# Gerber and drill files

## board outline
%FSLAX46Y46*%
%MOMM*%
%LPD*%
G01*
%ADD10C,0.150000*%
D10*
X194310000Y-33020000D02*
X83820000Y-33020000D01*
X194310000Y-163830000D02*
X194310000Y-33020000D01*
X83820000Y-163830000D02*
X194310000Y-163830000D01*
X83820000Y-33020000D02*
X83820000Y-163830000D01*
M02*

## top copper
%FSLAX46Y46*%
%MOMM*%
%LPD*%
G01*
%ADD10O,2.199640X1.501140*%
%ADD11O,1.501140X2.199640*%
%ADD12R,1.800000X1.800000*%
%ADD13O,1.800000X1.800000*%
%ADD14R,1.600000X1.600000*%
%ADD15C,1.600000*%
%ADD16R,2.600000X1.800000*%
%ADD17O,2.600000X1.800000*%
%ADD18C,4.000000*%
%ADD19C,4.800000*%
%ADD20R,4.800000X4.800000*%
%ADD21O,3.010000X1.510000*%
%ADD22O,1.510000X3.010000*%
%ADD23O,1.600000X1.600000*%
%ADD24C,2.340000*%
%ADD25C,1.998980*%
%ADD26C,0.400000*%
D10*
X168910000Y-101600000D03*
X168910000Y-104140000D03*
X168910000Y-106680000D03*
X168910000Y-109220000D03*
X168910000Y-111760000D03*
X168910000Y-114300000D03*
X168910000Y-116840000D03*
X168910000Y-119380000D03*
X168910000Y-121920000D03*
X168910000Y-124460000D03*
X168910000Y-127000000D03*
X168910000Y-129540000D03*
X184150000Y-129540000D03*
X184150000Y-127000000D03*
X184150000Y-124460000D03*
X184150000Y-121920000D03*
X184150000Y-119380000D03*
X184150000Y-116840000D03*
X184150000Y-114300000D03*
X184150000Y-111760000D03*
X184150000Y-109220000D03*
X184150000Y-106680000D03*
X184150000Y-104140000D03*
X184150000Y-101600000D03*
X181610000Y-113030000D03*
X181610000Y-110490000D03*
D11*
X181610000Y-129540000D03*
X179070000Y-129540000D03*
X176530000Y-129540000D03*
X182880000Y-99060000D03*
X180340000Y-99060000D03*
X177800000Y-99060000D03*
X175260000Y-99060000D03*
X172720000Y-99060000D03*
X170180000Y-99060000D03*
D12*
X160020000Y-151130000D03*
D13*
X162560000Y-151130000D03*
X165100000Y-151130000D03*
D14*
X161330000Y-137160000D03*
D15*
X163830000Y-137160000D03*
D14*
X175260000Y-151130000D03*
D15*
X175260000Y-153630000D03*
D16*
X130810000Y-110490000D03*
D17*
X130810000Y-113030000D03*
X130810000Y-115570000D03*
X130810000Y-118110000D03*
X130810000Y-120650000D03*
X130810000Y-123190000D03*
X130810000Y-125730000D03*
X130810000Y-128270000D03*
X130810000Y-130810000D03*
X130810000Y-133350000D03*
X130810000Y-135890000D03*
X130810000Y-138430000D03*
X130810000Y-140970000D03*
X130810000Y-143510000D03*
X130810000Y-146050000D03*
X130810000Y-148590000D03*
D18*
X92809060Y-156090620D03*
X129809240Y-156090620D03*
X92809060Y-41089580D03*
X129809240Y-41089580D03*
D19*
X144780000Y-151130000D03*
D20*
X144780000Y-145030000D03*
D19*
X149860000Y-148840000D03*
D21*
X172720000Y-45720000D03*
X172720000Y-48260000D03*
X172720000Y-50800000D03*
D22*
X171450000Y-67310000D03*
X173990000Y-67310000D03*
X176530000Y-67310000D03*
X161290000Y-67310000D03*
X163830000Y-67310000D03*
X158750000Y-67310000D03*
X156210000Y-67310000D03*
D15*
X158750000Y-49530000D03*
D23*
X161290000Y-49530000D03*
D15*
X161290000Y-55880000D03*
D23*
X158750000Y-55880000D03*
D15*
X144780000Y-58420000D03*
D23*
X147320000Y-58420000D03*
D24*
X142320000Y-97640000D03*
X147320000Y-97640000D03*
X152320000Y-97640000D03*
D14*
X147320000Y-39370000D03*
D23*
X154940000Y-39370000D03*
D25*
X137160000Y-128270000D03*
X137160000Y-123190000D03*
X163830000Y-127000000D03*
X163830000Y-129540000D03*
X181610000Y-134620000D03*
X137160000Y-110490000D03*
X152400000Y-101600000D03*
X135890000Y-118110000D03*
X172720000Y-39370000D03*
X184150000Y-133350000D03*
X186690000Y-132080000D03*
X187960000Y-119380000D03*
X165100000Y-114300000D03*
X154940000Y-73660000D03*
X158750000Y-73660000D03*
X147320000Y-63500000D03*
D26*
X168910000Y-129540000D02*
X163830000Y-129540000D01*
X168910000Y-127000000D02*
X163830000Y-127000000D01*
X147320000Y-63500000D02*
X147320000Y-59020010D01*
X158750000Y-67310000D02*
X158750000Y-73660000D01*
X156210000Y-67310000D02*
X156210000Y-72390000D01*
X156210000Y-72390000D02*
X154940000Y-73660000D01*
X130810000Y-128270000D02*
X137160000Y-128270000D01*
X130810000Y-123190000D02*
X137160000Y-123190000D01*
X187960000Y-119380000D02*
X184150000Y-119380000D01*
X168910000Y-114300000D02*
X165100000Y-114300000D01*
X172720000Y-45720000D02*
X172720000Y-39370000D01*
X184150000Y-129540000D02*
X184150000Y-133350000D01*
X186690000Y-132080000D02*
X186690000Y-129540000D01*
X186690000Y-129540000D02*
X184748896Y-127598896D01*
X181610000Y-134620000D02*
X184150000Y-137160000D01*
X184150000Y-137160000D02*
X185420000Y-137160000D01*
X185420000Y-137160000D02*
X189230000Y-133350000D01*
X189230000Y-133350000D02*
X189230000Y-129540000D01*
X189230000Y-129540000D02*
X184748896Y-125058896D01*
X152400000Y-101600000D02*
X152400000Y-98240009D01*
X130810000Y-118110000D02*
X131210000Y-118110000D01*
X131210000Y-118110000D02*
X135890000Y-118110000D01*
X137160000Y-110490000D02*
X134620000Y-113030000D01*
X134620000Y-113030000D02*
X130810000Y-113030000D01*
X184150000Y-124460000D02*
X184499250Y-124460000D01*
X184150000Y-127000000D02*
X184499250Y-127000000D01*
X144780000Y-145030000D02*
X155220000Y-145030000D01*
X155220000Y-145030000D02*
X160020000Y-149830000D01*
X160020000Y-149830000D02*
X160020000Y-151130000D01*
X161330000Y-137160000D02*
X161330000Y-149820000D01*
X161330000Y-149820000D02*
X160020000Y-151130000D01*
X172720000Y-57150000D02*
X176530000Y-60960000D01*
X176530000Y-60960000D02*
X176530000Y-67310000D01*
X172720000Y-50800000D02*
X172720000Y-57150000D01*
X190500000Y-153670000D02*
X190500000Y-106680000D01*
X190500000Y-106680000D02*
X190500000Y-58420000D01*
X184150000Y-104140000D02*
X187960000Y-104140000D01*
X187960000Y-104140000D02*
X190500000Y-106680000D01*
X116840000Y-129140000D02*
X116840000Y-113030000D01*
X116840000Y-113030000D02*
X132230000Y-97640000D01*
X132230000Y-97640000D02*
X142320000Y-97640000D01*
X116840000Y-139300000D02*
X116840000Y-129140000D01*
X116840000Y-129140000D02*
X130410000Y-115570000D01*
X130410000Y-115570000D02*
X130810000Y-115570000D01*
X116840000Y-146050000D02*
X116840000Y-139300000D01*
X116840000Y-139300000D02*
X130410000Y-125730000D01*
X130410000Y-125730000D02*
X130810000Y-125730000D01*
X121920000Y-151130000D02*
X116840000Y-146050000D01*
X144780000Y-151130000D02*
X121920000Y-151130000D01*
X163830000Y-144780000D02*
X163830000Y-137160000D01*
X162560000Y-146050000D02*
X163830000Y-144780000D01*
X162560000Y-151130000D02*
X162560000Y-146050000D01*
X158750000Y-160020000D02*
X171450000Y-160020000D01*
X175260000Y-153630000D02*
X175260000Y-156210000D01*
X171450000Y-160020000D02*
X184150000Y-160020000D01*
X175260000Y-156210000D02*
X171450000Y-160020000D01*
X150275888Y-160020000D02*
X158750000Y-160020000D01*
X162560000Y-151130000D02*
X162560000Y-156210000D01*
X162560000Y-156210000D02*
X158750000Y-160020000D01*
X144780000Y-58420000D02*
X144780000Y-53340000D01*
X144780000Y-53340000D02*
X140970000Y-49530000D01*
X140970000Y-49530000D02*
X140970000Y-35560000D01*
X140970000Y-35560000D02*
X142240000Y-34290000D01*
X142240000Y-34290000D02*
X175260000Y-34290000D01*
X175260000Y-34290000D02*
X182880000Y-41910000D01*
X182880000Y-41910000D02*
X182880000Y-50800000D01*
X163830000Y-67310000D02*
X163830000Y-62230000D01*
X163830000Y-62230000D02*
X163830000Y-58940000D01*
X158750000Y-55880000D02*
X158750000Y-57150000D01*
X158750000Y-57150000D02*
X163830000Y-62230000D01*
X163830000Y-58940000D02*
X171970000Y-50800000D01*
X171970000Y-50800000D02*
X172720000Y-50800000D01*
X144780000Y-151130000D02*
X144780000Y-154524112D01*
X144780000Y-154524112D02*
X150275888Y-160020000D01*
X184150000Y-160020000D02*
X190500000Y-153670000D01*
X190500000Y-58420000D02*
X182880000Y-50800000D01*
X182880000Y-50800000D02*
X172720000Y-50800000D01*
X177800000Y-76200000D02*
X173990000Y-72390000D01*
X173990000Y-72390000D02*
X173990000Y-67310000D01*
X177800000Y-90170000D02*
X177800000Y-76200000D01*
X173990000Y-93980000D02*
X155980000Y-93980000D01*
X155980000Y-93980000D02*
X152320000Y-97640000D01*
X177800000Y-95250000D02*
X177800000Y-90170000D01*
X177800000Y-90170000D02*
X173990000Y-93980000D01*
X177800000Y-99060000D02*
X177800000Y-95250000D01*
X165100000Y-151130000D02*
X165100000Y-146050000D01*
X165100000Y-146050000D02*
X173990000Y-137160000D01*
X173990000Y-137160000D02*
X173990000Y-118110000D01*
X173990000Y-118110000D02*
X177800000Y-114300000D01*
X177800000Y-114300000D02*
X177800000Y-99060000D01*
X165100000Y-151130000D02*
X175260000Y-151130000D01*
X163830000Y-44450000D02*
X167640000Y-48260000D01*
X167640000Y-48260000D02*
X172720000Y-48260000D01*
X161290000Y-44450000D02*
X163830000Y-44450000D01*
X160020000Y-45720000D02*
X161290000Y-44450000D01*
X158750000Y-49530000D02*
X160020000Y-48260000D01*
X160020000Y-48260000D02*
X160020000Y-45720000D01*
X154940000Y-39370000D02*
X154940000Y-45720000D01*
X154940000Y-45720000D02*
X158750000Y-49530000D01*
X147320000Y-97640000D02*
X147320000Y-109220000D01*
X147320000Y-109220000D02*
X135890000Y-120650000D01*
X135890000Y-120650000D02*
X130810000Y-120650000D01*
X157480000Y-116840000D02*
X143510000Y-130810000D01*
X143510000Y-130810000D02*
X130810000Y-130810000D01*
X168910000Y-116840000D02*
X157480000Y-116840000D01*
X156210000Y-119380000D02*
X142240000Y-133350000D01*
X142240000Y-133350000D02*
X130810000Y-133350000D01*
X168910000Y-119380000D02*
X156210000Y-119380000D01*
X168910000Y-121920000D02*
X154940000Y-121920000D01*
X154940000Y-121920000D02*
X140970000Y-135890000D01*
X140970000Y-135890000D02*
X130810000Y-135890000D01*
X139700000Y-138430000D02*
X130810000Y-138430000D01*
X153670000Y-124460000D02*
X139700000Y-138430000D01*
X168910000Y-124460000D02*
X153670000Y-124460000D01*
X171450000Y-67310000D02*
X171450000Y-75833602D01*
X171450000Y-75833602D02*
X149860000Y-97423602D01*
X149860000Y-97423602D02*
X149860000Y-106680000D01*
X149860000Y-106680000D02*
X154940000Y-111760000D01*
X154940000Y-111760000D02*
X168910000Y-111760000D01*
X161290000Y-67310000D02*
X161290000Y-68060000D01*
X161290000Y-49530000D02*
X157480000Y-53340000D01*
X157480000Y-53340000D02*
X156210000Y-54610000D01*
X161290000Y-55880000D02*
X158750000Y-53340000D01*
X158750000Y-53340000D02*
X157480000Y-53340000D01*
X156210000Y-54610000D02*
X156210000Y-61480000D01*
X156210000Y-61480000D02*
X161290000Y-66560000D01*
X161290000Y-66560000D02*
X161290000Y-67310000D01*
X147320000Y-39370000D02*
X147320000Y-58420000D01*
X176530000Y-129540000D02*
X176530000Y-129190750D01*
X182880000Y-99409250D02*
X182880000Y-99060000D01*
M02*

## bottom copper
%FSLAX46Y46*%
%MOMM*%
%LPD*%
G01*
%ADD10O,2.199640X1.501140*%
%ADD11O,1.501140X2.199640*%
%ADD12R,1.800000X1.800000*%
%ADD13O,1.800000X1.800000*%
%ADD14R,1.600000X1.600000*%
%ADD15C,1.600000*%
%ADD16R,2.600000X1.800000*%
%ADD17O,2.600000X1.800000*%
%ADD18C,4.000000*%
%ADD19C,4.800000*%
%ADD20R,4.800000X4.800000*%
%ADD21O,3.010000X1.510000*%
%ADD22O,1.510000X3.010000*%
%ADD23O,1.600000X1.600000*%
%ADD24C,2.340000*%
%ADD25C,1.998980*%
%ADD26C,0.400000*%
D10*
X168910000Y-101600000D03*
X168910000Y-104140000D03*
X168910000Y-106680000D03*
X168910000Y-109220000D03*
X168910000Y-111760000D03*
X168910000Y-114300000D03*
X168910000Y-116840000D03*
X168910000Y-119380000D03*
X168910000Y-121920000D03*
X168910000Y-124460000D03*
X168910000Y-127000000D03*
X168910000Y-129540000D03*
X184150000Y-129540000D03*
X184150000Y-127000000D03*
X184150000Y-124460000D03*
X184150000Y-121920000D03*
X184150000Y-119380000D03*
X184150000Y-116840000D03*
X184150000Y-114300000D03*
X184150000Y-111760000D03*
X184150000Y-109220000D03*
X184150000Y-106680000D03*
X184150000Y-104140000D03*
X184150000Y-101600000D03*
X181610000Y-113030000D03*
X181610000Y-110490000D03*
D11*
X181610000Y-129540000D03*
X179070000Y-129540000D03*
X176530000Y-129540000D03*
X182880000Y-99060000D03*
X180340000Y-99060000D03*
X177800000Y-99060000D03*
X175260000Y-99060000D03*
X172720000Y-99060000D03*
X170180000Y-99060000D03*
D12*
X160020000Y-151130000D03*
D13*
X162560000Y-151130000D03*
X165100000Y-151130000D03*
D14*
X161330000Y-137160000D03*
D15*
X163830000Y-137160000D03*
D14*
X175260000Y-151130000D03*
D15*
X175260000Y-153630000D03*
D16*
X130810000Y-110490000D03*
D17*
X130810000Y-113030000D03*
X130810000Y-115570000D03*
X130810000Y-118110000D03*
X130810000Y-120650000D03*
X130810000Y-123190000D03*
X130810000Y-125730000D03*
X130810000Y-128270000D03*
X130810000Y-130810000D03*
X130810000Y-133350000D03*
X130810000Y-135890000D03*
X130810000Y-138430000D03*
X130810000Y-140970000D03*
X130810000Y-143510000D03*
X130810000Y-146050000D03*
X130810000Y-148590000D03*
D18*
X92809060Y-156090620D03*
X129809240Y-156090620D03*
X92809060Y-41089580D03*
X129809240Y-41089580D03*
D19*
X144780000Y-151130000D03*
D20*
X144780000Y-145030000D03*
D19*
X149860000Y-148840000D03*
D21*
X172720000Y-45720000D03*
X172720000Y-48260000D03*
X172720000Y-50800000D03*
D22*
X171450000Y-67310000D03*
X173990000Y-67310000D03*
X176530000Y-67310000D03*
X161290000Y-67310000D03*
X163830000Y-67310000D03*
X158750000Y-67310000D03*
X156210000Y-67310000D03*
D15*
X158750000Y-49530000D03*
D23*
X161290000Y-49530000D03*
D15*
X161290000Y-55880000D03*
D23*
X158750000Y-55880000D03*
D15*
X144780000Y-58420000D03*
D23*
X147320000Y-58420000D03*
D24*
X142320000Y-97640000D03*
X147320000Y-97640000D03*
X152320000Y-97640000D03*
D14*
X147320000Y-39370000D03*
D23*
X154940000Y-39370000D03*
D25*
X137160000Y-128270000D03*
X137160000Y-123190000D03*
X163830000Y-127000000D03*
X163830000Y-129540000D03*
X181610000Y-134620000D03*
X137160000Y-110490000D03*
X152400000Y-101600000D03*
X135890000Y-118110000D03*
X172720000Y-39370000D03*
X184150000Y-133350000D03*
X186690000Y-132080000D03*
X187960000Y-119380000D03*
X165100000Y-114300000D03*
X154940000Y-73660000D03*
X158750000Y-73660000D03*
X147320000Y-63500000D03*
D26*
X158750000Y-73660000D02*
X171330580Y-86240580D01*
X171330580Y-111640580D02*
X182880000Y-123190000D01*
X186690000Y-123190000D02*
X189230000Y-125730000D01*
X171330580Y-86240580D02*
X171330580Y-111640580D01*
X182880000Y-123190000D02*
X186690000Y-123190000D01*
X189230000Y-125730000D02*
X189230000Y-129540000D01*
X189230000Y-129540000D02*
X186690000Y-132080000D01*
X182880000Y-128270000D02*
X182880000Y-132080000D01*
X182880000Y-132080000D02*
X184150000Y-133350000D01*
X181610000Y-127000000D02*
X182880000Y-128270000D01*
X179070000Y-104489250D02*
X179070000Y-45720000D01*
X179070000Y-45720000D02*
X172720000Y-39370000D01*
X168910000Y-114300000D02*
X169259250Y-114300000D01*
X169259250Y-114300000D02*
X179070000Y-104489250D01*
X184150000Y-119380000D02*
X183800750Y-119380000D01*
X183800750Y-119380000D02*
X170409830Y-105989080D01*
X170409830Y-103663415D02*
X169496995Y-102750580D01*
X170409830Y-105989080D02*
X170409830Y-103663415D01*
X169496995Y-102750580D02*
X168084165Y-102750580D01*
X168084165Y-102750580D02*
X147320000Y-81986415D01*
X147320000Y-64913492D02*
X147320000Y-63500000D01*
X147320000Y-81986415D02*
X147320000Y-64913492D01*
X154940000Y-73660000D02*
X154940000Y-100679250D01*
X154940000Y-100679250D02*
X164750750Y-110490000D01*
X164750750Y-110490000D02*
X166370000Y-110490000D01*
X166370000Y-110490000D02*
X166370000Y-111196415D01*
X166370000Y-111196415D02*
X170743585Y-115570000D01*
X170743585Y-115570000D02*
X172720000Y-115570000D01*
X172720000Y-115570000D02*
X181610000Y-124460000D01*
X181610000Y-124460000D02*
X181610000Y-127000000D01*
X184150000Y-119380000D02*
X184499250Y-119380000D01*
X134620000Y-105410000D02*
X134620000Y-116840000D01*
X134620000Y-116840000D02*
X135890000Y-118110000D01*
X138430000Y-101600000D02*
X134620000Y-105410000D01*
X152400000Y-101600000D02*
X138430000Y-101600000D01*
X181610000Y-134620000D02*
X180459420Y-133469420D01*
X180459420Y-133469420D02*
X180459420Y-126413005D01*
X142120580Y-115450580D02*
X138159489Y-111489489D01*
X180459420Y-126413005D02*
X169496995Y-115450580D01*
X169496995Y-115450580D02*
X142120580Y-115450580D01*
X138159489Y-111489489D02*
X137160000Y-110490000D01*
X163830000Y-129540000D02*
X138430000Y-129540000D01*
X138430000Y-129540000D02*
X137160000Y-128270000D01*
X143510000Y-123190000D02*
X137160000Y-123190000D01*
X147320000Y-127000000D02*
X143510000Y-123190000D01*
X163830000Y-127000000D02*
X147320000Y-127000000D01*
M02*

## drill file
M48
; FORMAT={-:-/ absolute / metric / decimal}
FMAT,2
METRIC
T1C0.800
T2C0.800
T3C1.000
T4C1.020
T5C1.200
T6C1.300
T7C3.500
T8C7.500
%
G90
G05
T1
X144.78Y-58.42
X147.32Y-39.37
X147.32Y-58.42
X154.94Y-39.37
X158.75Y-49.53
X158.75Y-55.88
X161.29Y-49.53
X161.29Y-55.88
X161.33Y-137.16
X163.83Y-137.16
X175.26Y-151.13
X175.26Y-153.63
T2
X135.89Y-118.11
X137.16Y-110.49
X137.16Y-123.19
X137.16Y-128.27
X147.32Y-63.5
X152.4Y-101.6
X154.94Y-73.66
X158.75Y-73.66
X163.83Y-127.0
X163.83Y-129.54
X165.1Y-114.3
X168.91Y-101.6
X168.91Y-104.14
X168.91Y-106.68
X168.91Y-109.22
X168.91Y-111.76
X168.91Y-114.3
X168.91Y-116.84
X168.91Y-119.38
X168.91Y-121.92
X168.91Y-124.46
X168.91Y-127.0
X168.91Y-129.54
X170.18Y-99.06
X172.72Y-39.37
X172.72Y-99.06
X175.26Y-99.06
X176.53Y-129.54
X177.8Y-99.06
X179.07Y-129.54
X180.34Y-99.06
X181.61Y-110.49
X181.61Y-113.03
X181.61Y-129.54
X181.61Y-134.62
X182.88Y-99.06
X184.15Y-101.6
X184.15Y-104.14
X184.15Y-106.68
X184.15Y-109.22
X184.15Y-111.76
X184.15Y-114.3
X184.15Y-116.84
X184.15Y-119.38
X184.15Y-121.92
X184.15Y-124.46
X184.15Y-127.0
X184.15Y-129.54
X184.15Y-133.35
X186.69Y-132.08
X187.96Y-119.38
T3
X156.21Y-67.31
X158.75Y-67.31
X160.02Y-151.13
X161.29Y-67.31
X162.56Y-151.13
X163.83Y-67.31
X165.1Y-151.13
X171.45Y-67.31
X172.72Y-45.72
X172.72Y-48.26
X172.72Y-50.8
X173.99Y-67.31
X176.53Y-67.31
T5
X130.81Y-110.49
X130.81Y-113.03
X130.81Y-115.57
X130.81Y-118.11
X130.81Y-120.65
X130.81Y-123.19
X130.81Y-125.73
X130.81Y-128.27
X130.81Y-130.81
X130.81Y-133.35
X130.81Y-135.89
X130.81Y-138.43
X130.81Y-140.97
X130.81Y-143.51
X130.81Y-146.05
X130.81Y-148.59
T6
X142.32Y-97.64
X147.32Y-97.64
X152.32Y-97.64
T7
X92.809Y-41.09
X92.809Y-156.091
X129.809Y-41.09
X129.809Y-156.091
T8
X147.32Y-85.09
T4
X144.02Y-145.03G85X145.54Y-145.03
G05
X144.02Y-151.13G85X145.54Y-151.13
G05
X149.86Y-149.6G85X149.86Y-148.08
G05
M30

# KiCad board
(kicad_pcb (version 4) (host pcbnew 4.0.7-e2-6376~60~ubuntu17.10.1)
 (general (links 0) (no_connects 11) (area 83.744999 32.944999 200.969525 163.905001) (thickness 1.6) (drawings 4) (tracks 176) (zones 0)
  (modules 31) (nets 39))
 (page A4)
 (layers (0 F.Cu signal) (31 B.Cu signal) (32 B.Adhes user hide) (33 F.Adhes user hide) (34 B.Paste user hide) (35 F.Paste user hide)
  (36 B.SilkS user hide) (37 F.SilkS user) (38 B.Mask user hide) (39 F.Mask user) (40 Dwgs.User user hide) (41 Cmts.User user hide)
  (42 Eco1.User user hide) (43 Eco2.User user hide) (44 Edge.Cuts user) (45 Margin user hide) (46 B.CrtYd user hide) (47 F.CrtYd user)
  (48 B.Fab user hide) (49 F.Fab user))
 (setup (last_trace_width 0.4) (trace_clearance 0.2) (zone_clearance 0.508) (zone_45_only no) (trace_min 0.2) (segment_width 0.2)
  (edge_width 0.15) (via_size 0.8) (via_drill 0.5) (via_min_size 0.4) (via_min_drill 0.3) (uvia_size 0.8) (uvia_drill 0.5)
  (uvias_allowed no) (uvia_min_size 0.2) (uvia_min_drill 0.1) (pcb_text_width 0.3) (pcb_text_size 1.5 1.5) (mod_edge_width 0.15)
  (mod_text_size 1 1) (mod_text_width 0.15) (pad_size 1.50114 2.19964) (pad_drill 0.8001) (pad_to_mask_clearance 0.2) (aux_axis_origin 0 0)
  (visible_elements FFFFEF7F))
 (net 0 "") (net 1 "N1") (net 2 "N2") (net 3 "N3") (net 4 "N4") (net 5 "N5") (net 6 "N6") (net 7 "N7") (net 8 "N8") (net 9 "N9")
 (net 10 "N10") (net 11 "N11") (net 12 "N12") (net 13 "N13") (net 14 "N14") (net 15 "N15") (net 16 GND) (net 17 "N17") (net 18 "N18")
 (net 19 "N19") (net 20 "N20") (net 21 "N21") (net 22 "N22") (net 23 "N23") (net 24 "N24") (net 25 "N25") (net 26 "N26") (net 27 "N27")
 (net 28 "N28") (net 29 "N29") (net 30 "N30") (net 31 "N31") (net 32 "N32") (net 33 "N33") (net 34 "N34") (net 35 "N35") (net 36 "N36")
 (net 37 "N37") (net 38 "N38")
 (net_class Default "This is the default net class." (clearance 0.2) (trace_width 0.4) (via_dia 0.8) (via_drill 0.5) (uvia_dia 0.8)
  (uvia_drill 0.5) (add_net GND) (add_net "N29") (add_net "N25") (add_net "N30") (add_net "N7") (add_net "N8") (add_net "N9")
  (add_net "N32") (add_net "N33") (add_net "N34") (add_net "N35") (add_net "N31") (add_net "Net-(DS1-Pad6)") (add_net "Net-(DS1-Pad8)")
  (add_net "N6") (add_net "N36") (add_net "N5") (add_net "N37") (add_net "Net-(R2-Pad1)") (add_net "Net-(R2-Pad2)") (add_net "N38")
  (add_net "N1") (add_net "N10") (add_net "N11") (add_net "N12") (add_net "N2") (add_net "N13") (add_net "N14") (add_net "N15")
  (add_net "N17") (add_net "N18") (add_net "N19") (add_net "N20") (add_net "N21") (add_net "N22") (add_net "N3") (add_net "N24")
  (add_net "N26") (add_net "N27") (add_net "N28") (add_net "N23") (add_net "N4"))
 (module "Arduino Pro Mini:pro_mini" (layer F.Cu) (at 176.53 115.57 270)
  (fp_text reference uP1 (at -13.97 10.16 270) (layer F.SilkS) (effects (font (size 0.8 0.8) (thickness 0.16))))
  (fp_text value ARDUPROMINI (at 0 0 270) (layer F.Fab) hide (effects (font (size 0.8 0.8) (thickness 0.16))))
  (pad 1 thru_hole oval (at -13.97 7.62 270) (size 1.50114 2.19964) (drill 0.8001) (layers *.Cu *.Mask F.SilkS) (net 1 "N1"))
  (pad 2 thru_hole oval (at -11.43 7.62 270) (size 1.50114 2.19964) (drill 0.8001) (layers *.Cu *.Mask F.SilkS) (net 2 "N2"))
  (pad 3 thru_hole oval (at -8.89 7.62 270) (size 1.50114 2.19964) (drill 0.8001) (layers *.Cu *.Mask F.SilkS) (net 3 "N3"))
  (pad 4 thru_hole oval (at -6.35 7.62 270) (size 1.50114 2.19964) (drill 0.8001) (layers *.Cu *.Mask F.SilkS) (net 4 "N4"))
  (pad 5 thru_hole oval (at -3.81 7.62 270) (size 1.50114 2.19964) (drill 0.8001) (layers *.Cu *.Mask F.SilkS) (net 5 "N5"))
  (pad 6 thru_hole oval (at -1.27 7.62 270) (size 1.50114 2.19964) (drill 0.8001) (layers *.Cu *.Mask F.SilkS))
  (pad 7 thru_hole oval (at 1.27 7.62 270) (size 1.50114 2.19964) (drill 0.8001) (layers *.Cu *.Mask F.SilkS) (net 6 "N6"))
  (pad 8 thru_hole oval (at 3.81 7.62 270) (size 1.50114 2.19964) (drill 0.8001) (layers *.Cu *.Mask F.SilkS) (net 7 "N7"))
  (pad 9 thru_hole oval (at 6.35 7.62 270) (size 1.50114 2.19964) (drill 0.8001) (layers *.Cu *.Mask F.SilkS) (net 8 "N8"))
  (pad 10 thru_hole oval (at 8.89 7.62 270) (size 1.50114 2.19964) (drill 0.8001) (layers *.Cu *.Mask F.SilkS) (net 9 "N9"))
  (pad 11 thru_hole oval (at 11.43 7.62 270) (size 1.50114 2.19964) (drill 0.8001) (layers *.Cu *.Mask F.SilkS))
  (pad 12 thru_hole oval (at 13.97 7.62 270) (size 1.50114 2.19964) (drill 0.8001) (layers *.Cu *.Mask F.SilkS))
  (pad 13 thru_hole oval (at 13.97 -7.62 270) (size 1.50114 2.19964) (drill 0.8001) (layers *.Cu *.Mask F.SilkS))
  (pad 14 thru_hole oval (at 11.43 -7.62 270) (size 1.50114 2.19964) (drill 0.8001) (layers *.Cu *.Mask F.SilkS))
  (pad 15 thru_hole oval (at 8.89 -7.62 270) (size 1.50114 2.19964) (drill 0.8001) (layers *.Cu *.Mask F.SilkS))
  (pad 16 thru_hole oval (at 6.35 -7.62 270) (size 1.50114 2.19964) (drill 0.8001) (layers *.Cu *.Mask F.SilkS) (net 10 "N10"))
  (pad 17 thru_hole oval (at 3.81 -7.62 270) (size 1.50114 2.19964) (drill 0.8001) (layers *.Cu *.Mask F.SilkS))
  (pad 18 thru_hole oval (at 1.27 -7.62 270) (size 1.50114 2.19964) (drill 0.8001) (layers *.Cu *.Mask F.SilkS) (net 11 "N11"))
  (pad 19 thru_hole oval (at -1.27 -7.62 270) (size 1.50114 2.19964) (drill 0.8001) (layers *.Cu *.Mask F.SilkS) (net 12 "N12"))
  (pad 20 thru_hole oval (at -3.81 -7.62 270) (size 1.50114 2.19964) (drill 0.8001) (layers *.Cu *.Mask F.SilkS) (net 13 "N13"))
  (pad 21 thru_hole oval (at -6.35 -7.62 270) (size 1.50114 2.19964) (drill 0.8001) (layers *.Cu *.Mask F.SilkS) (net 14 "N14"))
  (pad 22 thru_hole oval (at -8.89 -7.62 270) (size 1.50114 2.19964) (drill 0.8001) (layers *.Cu *.Mask F.SilkS) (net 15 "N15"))
  (pad 23 thru_hole oval (at -11.43 -7.62 270) (size 1.50114 2.19964) (drill 0.8001) (layers *.Cu *.Mask F.SilkS) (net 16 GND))
  (pad 24 thru_hole oval (at -13.97 -7.62 270) (size 1.50114 2.19964) (drill 0.8001) (layers *.Cu *.Mask F.SilkS) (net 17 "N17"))
  (pad 25 thru_hole oval (at -2.54 -5.08 270) (size 1.50114 2.19964) (drill 0.8001) (layers *.Cu *.Mask F.SilkS) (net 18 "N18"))
  (pad 26 thru_hole oval (at -5.08 -5.08 270) (size 1.50114 2.19964) (drill 0.8001) (layers *.Cu *.Mask F.SilkS) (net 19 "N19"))
  (pad 27 thru_hole oval (at 13.97 -5.08 270) (size 2.19964 1.50114) (drill 0.8001) (layers *.Cu *.Mask F.SilkS) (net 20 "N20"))
  (pad 28 thru_hole oval (at 13.97 -2.54 270) (size 2.19964 1.50114) (drill 0.8001) (layers *.Cu *.Mask F.SilkS) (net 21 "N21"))
  (pad 29 thru_hole oval (at 13.97 0 270) (size 2.19964 1.50114) (drill 0.8001) (layers *.Cu *.Mask F.SilkS) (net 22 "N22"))
  (pad 35 thru_hole oval (at -16.51 -6.35) (size 1.50114 2.19964) (drill 0.8001) (layers *.Cu *.Mask F.SilkS) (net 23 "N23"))
  (pad 30 thru_hole oval (at -16.51 -3.81) (size 1.50114 2.19964) (drill 0.8001) (layers *.Cu *.Mask F.SilkS) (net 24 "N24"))
  (pad 31 thru_hole oval (at -16.51 -1.27) (size 1.50114 2.19964) (drill 0.8001) (layers *.Cu *.Mask F.SilkS) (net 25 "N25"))
  (pad 32 thru_hole oval (at -16.51 1.27) (size 1.50114 2.19964) (drill 0.8001) (layers *.Cu *.Mask F.SilkS) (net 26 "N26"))
  (pad 33 thru_hole oval (at -16.51 3.81) (size 1.50114 2.19964) (drill 0.8001) (layers *.Cu *.Mask F.SilkS) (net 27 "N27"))
  (pad 34 thru_hole oval (at -16.51 6.35) (size 1.50114 2.19964) (drill 0.8001) (layers *.Cu *.Mask F.SilkS) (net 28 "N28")))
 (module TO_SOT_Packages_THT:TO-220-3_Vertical (layer F.Cu) (at 160.02 151.13)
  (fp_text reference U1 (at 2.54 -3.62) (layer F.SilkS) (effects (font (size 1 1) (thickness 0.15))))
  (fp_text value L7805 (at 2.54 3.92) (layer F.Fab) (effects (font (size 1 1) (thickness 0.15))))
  (pad 1 thru_hole rect (at 0 0) (size 1.8 1.8) (drill 1) (layers *.Cu *.Mask) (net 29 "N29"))
  (pad 2 thru_hole oval (at 2.54 0) (size 1.8 1.8) (drill 1) (layers *.Cu *.Mask) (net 16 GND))
  (pad 3 thru_hole oval (at 5.08 0) (size 1.8 1.8) (drill 1) (layers *.Cu *.Mask) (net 25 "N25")))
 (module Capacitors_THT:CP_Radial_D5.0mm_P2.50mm (layer F.Cu) (at 161.33 137.16)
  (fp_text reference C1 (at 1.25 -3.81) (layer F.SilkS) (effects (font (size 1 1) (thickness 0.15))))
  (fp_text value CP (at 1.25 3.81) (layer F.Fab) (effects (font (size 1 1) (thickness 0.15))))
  (pad 1 thru_hole rect (at 0 0) (size 1.6 1.6) (drill 0.8) (layers *.Cu *.Mask) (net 29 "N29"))
  (pad 2 thru_hole circle (at 2.5 0) (size 1.6 1.6) (drill 0.8) (layers *.Cu *.Mask) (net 16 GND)))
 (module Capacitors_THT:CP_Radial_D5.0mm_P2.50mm (layer F.Cu) (at 175.26 151.13 270)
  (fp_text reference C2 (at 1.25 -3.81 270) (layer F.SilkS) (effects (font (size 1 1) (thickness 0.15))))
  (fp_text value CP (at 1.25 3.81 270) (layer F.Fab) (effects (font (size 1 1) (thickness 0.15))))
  (pad 1 thru_hole rect (at 0 0 270) (size 1.6 1.6) (drill 0.8) (layers *.Cu *.Mask) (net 25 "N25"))
  (pad 2 thru_hole circle (at 2.5 0 270) (size 1.6 1.6) (drill 0.8) (layers *.Cu *.Mask) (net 16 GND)))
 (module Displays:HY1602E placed (layer F.Cu) (at 130.81 110.49 270)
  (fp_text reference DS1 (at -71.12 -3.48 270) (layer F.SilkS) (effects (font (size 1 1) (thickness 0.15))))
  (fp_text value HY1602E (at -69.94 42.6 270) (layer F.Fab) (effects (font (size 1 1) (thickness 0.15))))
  (pad 1 thru_hole rect (at 0 0 90) (size 1.8 2.6) (drill 1.2) (layers *.Cu *.Mask) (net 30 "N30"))
  (pad 2 thru_hole oval (at 2.54 0 90) (size 1.8 2.6) (drill 1.2) (layers *.Cu *.Mask))
  (pad 3 thru_hole oval (at 5.08 0 90) (size 1.8 2.6) (drill 1.2) (layers *.Cu *.Mask) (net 16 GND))
  (pad 4 thru_hole oval (at 7.62 0 90) (size 1.8 2.6) (drill 1.2) (layers *.Cu *.Mask))
  (pad 5 thru_hole oval (at 10.16 0 90) (size 1.8 2.6) (drill 1.2) (layers *.Cu *.Mask) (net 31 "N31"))
  (pad 6 thru_hole oval (at 12.7 0 90) (size 1.8 2.6) (drill 1.2) (layers *.Cu *.Mask))
  (pad 7 thru_hole oval (at 15.24 0 90) (size 1.8 2.6) (drill 1.2) (layers *.Cu *.Mask) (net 16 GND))
  (pad 8 thru_hole oval (at 17.78 0 90) (size 1.8 2.6) (drill 1.2) (layers *.Cu *.Mask))
  (pad 9 thru_hole oval (at 20.32 0 90) (size 1.8 2.6) (drill 1.2) (layers *.Cu *.Mask) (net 6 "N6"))
  (pad 10 thru_hole oval (at 22.86 0 90) (size 1.8 2.6) (drill 1.2) (layers *.Cu *.Mask) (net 7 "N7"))
  (pad 11 thru_hole oval (at 25.4 0 90) (size 1.8 2.6) (drill 1.2) (layers *.Cu *.Mask) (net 8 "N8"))
  (pad 12 thru_hole oval (at 27.94 0 90) (size 1.8 2.6) (drill 1.2) (layers *.Cu *.Mask) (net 9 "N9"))
  (pad 13 thru_hole oval (at 30.48 0 90) (size 1.8 2.6) (drill 1.2) (layers *.Cu *.Mask) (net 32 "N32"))
  (pad 14 thru_hole oval (at 33.02 0 90) (size 1.8 2.6) (drill 1.2) (layers *.Cu *.Mask) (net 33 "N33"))
  (pad 15 thru_hole oval (at 35.56 0 90) (size 1.8 2.6) (drill 1.2) (layers *.Cu *.Mask) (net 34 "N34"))
  (pad 16 thru_hole oval (at 38.1 0 90) (size 1.8 2.6) (drill 1.2) (layers *.Cu *.Mask) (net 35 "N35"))
  (pad "" thru_hole circle (at 45.60062 38.00094 90) (size 4 4) (drill 3.5) (layers *.Cu *.Mask))
  (pad "" thru_hole circle (at 45.60062 1.00076 90) (size 4 4) (drill 3.5) (layers *.Cu *.Mask))
  (pad "" thru_hole circle (at -69.40042 38.00094 90) (size 4 4) (drill 3.5) (layers *.Cu *.Mask))
  (pad "" thru_hole circle (at -69.40042 1.00076 90) (size 4 4) (drill 3.5) (layers *.Cu *.Mask)))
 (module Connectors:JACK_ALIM (layer F.Cu) (at 144.78 145.03 90)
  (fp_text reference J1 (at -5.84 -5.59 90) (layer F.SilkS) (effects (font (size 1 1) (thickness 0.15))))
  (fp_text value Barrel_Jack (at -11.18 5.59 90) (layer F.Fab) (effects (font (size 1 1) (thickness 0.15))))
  (pad 2 thru_hole circle (at -6.1 0 90) (size 4.8 4.8) (drill oval 1.02 2.54) (layers *.Cu *.Mask) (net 16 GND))
  (pad 1 thru_hole rect (at 0 0 90) (size 4.8 4.8) (drill oval 1.02 2.54) (layers *.Cu *.Mask) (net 29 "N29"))
  (pad 3 thru_hole circle (at -3.81 5.08 90) (size 4.8 4.8) (drill oval 2.54 1.02) (layers *.Cu *.Mask) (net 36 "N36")))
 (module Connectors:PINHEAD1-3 (layer F.Cu) (at 172.72 45.72 270)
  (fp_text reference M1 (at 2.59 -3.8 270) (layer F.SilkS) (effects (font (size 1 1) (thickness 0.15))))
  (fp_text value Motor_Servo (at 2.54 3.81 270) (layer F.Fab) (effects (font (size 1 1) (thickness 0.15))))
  (pad 1 thru_hole oval (at 0 0 270) (size 1.51 3.01) (drill 1) (layers *.Cu *.Mask))
  (pad 2 thru_hole oval (at 2.54 0 270) (size 1.51 3.01) (drill 1) (layers *.Cu *.Mask) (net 25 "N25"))
  (pad 3 thru_hole oval (at 5.08 0 270) (size 1.51 3.01) (drill 1) (layers *.Cu *.Mask) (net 16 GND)))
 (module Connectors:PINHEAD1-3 (layer F.Cu) (at 171.45 67.31)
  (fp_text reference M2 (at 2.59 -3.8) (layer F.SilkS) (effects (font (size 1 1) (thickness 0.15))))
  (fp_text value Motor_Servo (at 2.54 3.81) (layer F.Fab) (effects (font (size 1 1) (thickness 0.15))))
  (pad 1 thru_hole oval (at 0 0) (size 1.51 3.01) (drill 1) (layers *.Cu *.Mask) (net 5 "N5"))
  (pad 2 thru_hole oval (at 2.54 0) (size 1.51 3.01) (drill 1) (layers *.Cu *.Mask) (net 25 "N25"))
  (pad 3 thru_hole oval (at 5.08 0) (size 1.51 3.01) (drill 1) (layers *.Cu *.Mask) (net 16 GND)))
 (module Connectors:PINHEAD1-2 (layer F.Cu) (at 161.29 67.31)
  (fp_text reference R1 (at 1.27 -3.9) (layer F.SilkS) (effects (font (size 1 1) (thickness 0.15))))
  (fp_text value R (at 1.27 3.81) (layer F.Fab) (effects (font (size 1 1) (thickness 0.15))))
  (pad 1 thru_hole oval (at 0 0) (size 1.51 3.01) (drill 1) (layers *.Cu *.Mask) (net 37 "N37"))
  (pad 2 thru_hole oval (at 2.54 0) (size 1.51 3.01) (drill 1) (layers *.Cu *.Mask) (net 16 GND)))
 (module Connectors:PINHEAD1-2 (layer F.Cu) (at 158.75 67.31 180)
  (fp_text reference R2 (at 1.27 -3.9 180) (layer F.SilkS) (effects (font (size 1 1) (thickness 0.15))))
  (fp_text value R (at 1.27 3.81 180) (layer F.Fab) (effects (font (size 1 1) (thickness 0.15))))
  (pad 1 thru_hole oval (at 0 0 180) (size 1.51 3.01) (drill 1) (layers *.Cu *.Mask))
  (pad 2 thru_hole oval (at 2.54 0 180) (size 1.51 3.01) (drill 1) (layers *.Cu *.Mask)))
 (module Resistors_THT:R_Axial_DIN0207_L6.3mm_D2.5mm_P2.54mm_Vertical (layer F.Cu) (at 158.75 49.53)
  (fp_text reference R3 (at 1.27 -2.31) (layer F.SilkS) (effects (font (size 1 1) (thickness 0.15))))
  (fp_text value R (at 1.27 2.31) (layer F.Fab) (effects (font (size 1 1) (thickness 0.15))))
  (pad 1 thru_hole circle (at 0 0) (size 1.6 1.6) (drill 0.8) (layers *.Cu *.Mask) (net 25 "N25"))
  (pad 2 thru_hole oval (at 2.54 0) (size 1.6 1.6) (drill 0.8) (layers *.Cu *.Mask) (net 37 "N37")))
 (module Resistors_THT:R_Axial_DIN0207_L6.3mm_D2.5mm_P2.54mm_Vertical (layer F.Cu) (at 161.29 55.88 180)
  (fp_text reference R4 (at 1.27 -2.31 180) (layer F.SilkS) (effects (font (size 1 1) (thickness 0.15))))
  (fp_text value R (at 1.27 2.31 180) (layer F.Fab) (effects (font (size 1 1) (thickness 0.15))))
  (pad 1 thru_hole circle (at 0 0 180) (size 1.6 1.6) (drill 0.8) (layers *.Cu *.Mask) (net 37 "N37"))
  (pad 2 thru_hole oval (at 2.54 0 180) (size 1.6 1.6) (drill 0.8) (layers *.Cu *.Mask) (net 16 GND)))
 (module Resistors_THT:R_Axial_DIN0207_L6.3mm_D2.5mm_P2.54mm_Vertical (layer F.Cu) (at 144.78 58.42)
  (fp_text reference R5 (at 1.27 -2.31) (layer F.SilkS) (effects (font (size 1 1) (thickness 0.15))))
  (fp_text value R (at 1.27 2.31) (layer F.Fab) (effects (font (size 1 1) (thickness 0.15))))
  (pad 1 thru_hole circle (at 0 0) (size 1.6 1.6) (drill 0.8) (layers *.Cu *.Mask) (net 16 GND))
  (pad 2 thru_hole oval (at 2.54 0) (size 1.6 1.6) (drill 0.8) (layers *.Cu *.Mask)))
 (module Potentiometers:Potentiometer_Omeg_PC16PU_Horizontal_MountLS (layer F.Cu) (at 152.32 97.64 90)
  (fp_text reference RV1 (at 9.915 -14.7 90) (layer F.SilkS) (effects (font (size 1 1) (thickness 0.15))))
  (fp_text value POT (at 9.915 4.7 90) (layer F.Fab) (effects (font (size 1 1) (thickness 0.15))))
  (pad 3 thru_hole circle (at 0 -10 90) (size 2.34 2.34) (drill 1.3) (layers *.Cu *.Mask) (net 16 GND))
  (pad 2 thru_hole circle (at 0 -5 90) (size 2.34 2.34) (drill 1.3) (layers *.Cu *.Mask) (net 31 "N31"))
  (pad 1 thru_hole circle (at 0 0 90) (size 2.34 2.34) (drill 1.3) (layers *.Cu *.Mask))
  (pad 0 np_thru_hole circle (at 12.55 -5 90) (size 7.5 7.5) (drill 7.5) (layers *.Cu *.Mask)))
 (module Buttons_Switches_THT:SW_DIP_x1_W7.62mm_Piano (layer F.Cu) (at 147.32 39.37)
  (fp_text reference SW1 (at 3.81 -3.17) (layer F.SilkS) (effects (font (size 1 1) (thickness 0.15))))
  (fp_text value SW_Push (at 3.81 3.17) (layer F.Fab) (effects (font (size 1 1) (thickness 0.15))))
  (pad 1 thru_hole rect (at 0 0) (size 1.6 1.6) (drill 0.8) (layers *.Cu *.Mask) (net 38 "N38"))
  (pad 2 thru_hole oval (at 7.62 0) (size 1.6 1.6) (drill 0.8) (layers *.Cu *.Mask) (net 25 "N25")))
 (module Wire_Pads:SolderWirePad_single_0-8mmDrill (layer F.Cu) (at 137.16 128.27)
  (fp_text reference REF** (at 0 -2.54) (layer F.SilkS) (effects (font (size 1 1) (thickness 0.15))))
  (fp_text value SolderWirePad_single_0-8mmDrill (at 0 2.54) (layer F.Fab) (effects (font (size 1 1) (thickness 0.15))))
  (pad 1 thru_hole circle (at 0 0) (size 1.99898 1.99898) (drill 0.8001) (layers *.Cu *.Mask)))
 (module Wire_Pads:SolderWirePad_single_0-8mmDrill (layer F.Cu) (at 137.16 123.19)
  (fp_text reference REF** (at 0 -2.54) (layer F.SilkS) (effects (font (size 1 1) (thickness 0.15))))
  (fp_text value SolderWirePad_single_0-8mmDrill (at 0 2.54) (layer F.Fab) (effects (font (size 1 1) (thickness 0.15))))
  (pad 1 thru_hole circle (at 0 0) (size 1.99898 1.99898) (drill 0.8001) (layers *.Cu *.Mask)))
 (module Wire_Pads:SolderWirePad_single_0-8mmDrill (layer F.Cu) (at 163.83 127)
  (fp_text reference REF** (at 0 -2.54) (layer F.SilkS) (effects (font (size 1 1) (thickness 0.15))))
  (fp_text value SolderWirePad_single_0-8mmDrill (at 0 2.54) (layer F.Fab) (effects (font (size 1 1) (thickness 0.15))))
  (pad 1 thru_hole circle (at 0 0) (size 1.99898 1.99898) (drill 0.8001) (layers *.Cu *.Mask)))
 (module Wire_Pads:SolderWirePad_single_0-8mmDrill (layer F.Cu) (at 163.83 129.54)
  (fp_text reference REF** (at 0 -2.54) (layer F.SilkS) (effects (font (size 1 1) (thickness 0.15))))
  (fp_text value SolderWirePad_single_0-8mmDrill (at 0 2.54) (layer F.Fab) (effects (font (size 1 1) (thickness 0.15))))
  (pad 1 thru_hole circle (at 0 0) (size 1.99898 1.99898) (drill 0.8001) (layers *.Cu *.Mask)))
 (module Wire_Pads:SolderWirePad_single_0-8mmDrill (layer F.Cu) (at 181.61 134.62)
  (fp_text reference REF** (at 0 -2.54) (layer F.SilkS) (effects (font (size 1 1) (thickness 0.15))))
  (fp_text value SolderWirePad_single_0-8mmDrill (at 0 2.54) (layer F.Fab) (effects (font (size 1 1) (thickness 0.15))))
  (pad 1 thru_hole circle (at 0 0) (size 1.99898 1.99898) (drill 0.8001) (layers *.Cu *.Mask)))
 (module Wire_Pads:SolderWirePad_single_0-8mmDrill (layer F.Cu) (at 137.16 110.49)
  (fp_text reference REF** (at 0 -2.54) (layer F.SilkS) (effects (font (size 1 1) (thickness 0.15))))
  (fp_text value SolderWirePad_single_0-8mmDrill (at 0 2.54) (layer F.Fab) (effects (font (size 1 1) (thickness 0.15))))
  (pad 1 thru_hole circle (at 0 0) (size 1.99898 1.99898) (drill 0.8001) (layers *.Cu *.Mask)))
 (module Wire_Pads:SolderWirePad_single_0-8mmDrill (layer F.Cu) (at 152.4 101.6)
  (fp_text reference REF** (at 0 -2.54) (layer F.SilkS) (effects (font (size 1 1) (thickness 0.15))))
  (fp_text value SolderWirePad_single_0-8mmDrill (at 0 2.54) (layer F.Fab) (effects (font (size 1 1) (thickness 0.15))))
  (pad 1 thru_hole circle (at 0 0) (size 1.99898 1.99898) (drill 0.8001) (layers *.Cu *.Mask)))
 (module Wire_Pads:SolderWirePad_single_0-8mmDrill (layer F.Cu) (at 135.89 118.11)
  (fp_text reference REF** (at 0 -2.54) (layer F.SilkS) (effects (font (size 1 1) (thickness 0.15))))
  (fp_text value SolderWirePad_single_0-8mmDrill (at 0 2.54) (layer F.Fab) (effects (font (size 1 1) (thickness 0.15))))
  (pad 1 thru_hole circle (at 0 0) (size 1.99898 1.99898) (drill 0.8001) (layers *.Cu *.Mask)))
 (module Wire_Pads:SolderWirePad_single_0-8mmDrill (layer F.Cu) (at 172.72 39.37)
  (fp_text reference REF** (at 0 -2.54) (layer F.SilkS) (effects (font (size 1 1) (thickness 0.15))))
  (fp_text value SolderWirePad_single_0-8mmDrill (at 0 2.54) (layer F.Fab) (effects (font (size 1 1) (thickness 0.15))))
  (pad 1 thru_hole circle (at 0 0) (size 1.99898 1.99898) (drill 0.8001) (layers *.Cu *.Mask)))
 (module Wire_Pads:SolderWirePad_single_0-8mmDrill (layer F.Cu) (at 184.15 133.35)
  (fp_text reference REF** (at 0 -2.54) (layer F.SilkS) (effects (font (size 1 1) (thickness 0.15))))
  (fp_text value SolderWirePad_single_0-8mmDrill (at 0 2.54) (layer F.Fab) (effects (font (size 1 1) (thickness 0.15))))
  (pad 1 thru_hole circle (at 0 0) (size 1.99898 1.99898) (drill 0.8001) (layers *.Cu *.Mask)))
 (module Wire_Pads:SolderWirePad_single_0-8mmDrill (layer F.Cu) (at 186.69 132.08)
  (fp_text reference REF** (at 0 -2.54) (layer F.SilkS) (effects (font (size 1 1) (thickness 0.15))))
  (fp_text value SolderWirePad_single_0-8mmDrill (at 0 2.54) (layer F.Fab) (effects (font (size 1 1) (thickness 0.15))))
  (pad 1 thru_hole circle (at 0 0) (size 1.99898 1.99898) (drill 0.8001) (layers *.Cu *.Mask)))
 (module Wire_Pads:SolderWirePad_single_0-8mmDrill (layer F.Cu) (at 187.96 119.38)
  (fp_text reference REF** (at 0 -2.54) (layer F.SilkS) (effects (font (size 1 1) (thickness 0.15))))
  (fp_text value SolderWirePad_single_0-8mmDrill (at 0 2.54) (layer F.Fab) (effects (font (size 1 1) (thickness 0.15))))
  (pad 1 thru_hole circle (at 0 0) (size 1.99898 1.99898) (drill 0.8001) (layers *.Cu *.Mask)))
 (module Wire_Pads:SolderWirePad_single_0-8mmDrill (layer F.Cu) (at 165.1 114.3)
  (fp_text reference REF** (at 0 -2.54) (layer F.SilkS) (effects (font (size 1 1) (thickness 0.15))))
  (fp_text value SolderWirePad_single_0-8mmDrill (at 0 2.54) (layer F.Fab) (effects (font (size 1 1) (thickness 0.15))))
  (pad 1 thru_hole circle (at 0 0) (size 1.99898 1.99898) (drill 0.8001) (layers *.Cu *.Mask)))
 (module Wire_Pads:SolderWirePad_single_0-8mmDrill (layer F.Cu) (at 154.94 73.66)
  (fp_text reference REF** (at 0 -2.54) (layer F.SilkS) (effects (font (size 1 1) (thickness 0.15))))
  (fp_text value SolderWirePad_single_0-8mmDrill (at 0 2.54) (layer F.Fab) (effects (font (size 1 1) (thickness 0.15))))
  (pad 1 thru_hole circle (at 0 0) (size 1.99898 1.99898) (drill 0.8001) (layers *.Cu *.Mask)))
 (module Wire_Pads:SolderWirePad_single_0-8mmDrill (layer F.Cu) (at 158.75 73.66)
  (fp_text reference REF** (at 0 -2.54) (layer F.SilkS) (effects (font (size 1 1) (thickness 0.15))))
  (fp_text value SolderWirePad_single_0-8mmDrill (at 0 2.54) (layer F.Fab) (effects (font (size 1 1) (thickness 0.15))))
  (pad 1 thru_hole circle (at 0 0) (size 1.99898 1.99898) (drill 0.8001) (layers *.Cu *.Mask)))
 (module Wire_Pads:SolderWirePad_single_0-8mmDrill (layer F.Cu) (at 147.32 63.5)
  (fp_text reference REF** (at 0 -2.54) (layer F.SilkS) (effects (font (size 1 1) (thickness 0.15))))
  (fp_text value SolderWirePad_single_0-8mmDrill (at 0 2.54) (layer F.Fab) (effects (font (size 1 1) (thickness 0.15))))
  (pad 1 thru_hole circle (at 0 0) (size 1.99898 1.99898) (drill 0.8001) (layers *.Cu *.Mask)))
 (gr_line (start 194.31 33.02) (end 83.82 33.02) (angle 90) (layer Edge.Cuts) (width 0.15))
 (gr_line (start 194.31 163.83) (end 194.31 33.02) (angle 90) (layer Edge.Cuts) (width 0.15))
 (gr_line (start 83.82 163.83) (end 194.31 163.83) (angle 90) (layer Edge.Cuts) (width 0.15))
 (gr_line (start 83.82 33.02) (end 83.82 163.83) (angle 90) (layer Edge.Cuts) (width 0.15))
 (segment (start 168.91 129.54) (end 163.83 129.54) (width 0.4) (layer F.Cu) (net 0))
 (segment (start 168.91 127) (end 163.83 127) (width 0.4) (layer F.Cu) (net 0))
 (segment (start 147.32 63.5) (end 147.32 59.02001) (width 0.4) (layer F.Cu) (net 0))
 (segment (start 158.75 67.31) (end 158.75 73.66) (width 0.4) (layer F.Cu) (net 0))
 (segment (start 156.21 67.31) (end 156.21 72.39) (width 0.4) (layer F.Cu) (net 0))
 (segment (start 156.21 72.39) (end 154.94 73.66) (width 0.4) (layer F.Cu) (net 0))
 (segment (start 130.81 128.27) (end 137.16 128.27) (width 0.4) (layer F.Cu) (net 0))
 (segment (start 130.81 123.19) (end 137.16 123.19) (width 0.4) (layer F.Cu) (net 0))
 (segment (start 158.75 73.66) (end 171.33058 86.24058) (width 0.4) (layer B.Cu) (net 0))
 (segment (start 171.33058 111.64058) (end 182.88 123.19) (width 0.4) (layer B.Cu) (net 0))
 (segment (start 186.69 123.19) (end 189.23 125.73) (width 0.4) (layer B.Cu) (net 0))
 (segment (start 171.33058 86.24058) (end 171.33058 111.64058) (width 0.4) (layer B.Cu) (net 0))
 (segment (start 182.88 123.19) (end 186.69 123.19) (width 0.4) (layer B.Cu) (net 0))
 (segment (start 189.23 125.73) (end 189.23 129.54) (width 0.4) (layer B.Cu) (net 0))
 (segment (start 189.23 129.54) (end 186.69 132.08) (width 0.4) (layer B.Cu) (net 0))
 (segment (start 182.88 128.27) (end 182.88 132.08) (width 0.4) (layer B.Cu) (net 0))
 (segment (start 182.88 132.08) (end 184.15 133.35) (width 0.4) (layer B.Cu) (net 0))
 (segment (start 181.61 127) (end 182.88 128.27) (width 0.4) (layer B.Cu) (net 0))
 (segment (start 179.07 104.48925) (end 179.07 45.72) (width 0.4) (layer B.Cu) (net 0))
 (segment (start 179.07 45.72) (end 172.72 39.37) (width 0.4) (layer B.Cu) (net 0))
 (segment (start 168.91 114.3) (end 169.25925 114.3) (width 0.4) (layer B.Cu) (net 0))
 (segment (start 169.25925 114.3) (end 179.07 104.48925) (width 0.4) (layer B.Cu) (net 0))
 (segment (start 184.15 119.38) (end 183.80075 119.38) (width 0.4) (layer B.Cu) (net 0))
 (segment (start 183.80075 119.38) (end 170.40983 105.98908) (width 0.4) (layer B.Cu) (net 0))
 (segment (start 170.40983 103.663415) (end 169.496995 102.75058) (width 0.4) (layer B.Cu) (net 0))
 (segment (start 170.40983 105.98908) (end 170.40983 103.663415) (width 0.4) (layer B.Cu) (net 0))
 (segment (start 169.496995 102.75058) (end 168.084165 102.75058) (width 0.4) (layer B.Cu) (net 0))
 (segment (start 168.084165 102.75058) (end 147.32 81.986415) (width 0.4) (layer B.Cu) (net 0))
 (segment (start 147.32 64.913492) (end 147.32 63.5) (width 0.4) (layer B.Cu) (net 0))
 (segment (start 147.32 81.986415) (end 147.32 64.913492) (width 0.4) (layer B.Cu) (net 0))
 (segment (start 154.94 73.66) (end 154.94 100.67925) (width 0.4) (layer B.Cu) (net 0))
 (segment (start 154.94 100.67925) (end 164.75075 110.49) (width 0.4) (layer B.Cu) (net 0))
 (segment (start 164.75075 110.49) (end 166.37 110.49) (width 0.4) (layer B.Cu) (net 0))
 (segment (start 166.37 110.49) (end 166.37 111.196415) (width 0.4) (layer B.Cu) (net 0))
 (segment (start 166.37 111.196415) (end 170.743585 115.57) (width 0.4) (layer B.Cu) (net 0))
 (segment (start 170.743585 115.57) (end 172.72 115.57) (width 0.4) (layer B.Cu) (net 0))
 (segment (start 172.72 115.57) (end 181.61 124.46) (width 0.4) (layer B.Cu) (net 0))
 (segment (start 181.61 124.46) (end 181.61 127) (width 0.4) (layer B.Cu) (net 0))
 (segment (start 184.15 119.38) (end 184.49925 119.38) (width 0.4) (layer B.Cu) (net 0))
 (segment (start 187.96 119.38) (end 184.15 119.38) (width 0.4) (layer F.Cu) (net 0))
 (segment (start 168.91 114.3) (end 165.1 114.3) (width 0.4) (layer F.Cu) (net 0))
 (segment (start 172.72 45.72) (end 172.72 39.37) (width 0.4) (layer F.Cu) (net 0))
 (segment (start 184.15 129.54) (end 184.15 133.35) (width 0.4) (layer F.Cu) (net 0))
 (segment (start 186.69 132.08) (end 186.69 129.54) (width 0.4) (layer F.Cu) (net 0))
 (segment (start 186.69 129.54) (end 184.748896 127.598896) (width 0.4) (layer F.Cu) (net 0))
 (segment (start 181.61 134.62) (end 184.15 137.16) (width 0.4) (layer F.Cu) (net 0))
 (segment (start 184.15 137.16) (end 185.42 137.16) (width 0.4) (layer F.Cu) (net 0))
 (segment (start 185.42 137.16) (end 189.23 133.35) (width 0.4) (layer F.Cu) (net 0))
 (segment (start 189.23 133.35) (end 189.23 129.54) (width 0.4) (layer F.Cu) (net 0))
 (segment (start 189.23 129.54) (end 184.748896 125.058896) (width 0.4) (layer F.Cu) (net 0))
 (segment (start 134.62 105.41) (end 134.62 116.84) (width 0.4) (layer B.Cu) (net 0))
 (segment (start 134.62 116.84) (end 135.89 118.11) (width 0.4) (layer B.Cu) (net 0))
 (segment (start 138.43 101.6) (end 134.62 105.41) (width 0.4) (layer B.Cu) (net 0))
 (segment (start 152.4 101.6) (end 138.43 101.6) (width 0.4) (layer B.Cu) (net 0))
 (segment (start 152.4 101.6) (end 152.4 98.240009) (width 0.4) (layer F.Cu) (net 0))
 (segment (start 130.81 118.11) (end 131.21 118.11) (width 0.4) (layer F.Cu) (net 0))
 (segment (start 131.21 118.11) (end 135.89 118.11) (width 0.4) (layer F.Cu) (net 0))
 (segment (start 137.16 110.49) (end 134.62 113.03) (width 0.4) (layer F.Cu) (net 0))
 (segment (start 134.62 113.03) (end 130.81 113.03) (width 0.4) (layer F.Cu) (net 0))
 (segment (start 181.61 134.62) (end 180.45942 133.46942) (width 0.4) (layer B.Cu) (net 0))
 (segment (start 180.45942 133.46942) (end 180.45942 126.413005) (width 0.4) (layer B.Cu) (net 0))
 (segment (start 142.12058 115.45058) (end 138.159489 111.489489) (width 0.4) (layer B.Cu) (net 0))
 (segment (start 180.45942 126.413005) (end 169.496995 115.45058) (width 0.4) (layer B.Cu) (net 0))
 (segment (start 169.496995 115.45058) (end 142.12058 115.45058) (width 0.4) (layer B.Cu) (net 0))
 (segment (start 138.159489 111.489489) (end 137.16 110.49) (width 0.4) (layer B.Cu) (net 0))
 (segment (start 163.83 129.54) (end 138.43 129.54) (width 0.4) (layer B.Cu) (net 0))
 (segment (start 138.43 129.54) (end 137.16 128.27) (width 0.4) (layer B.Cu) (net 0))
 (segment (start 143.51 123.19) (end 137.16 123.19) (width 0.4) (layer B.Cu) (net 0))
 (segment (start 147.32 127) (end 143.51 123.19) (width 0.4) (layer B.Cu) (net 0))
 (segment (start 163.83 127) (end 147.32 127) (width 0.4) (layer B.Cu) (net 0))
 (segment (start 184.15 124.46) (end 184.49925 124.46) (width 0.4) (layer F.Cu) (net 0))
 (segment (start 184.15 127) (end 184.49925 127) (width 0.4) (layer F.Cu) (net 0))
 (segment (start 144.78 145.03) (end 155.22 145.03) (width 0.4) (layer F.Cu) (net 29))
 (segment (start 155.22 145.03) (end 160.02 149.83) (width 0.4) (layer F.Cu) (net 29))
 (segment (start 160.02 149.83) (end 160.02 151.13) (width 0.4) (layer F.Cu) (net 29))
 (segment (start 161.33 137.16) (end 161.33 149.82) (width 0.4) (layer F.Cu) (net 29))
 (segment (start 161.33 149.82) (end 160.02 151.13) (width 0.4) (layer F.Cu) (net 29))
 (segment (start 172.72 57.15) (end 176.53 60.96) (width 0.4) (layer F.Cu) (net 16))
 (segment (start 176.53 60.96) (end 176.53 67.31) (width 0.4) (layer F.Cu) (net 16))
 (segment (start 172.72 50.8) (end 172.72 57.15) (width 0.4) (layer F.Cu) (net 16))
 (segment (start 190.5 153.67) (end 190.5 106.68) (width 0.4) (layer F.Cu) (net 16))
 (segment (start 190.5 106.68) (end 190.5 58.42) (width 0.4) (layer F.Cu) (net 16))
 (segment (start 184.15 104.14) (end 187.96 104.14) (width 0.4) (layer F.Cu) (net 16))
 (segment (start 187.96 104.14) (end 190.5 106.68) (width 0.4) (layer F.Cu) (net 16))
 (segment (start 116.84 129.14) (end 116.84 113.03) (width 0.4) (layer F.Cu) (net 16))
 (segment (start 116.84 113.03) (end 132.23 97.64) (width 0.4) (layer F.Cu) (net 16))
 (segment (start 132.23 97.64) (end 142.32 97.64) (width 0.4) (layer F.Cu) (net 16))
 (segment (start 116.84 139.3) (end 116.84 129.14) (width 0.4) (layer F.Cu) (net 16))
 (segment (start 116.84 129.14) (end 130.41 115.57) (width 0.4) (layer F.Cu) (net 16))
 (segment (start 130.41 115.57) (end 130.81 115.57) (width 0.4) (layer F.Cu) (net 16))
 (segment (start 116.84 146.05) (end 116.84 139.3) (width 0.4) (layer F.Cu) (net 16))
 (segment (start 116.84 139.3) (end 130.41 125.73) (width 0.4) (layer F.Cu) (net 16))
 (segment (start 130.41 125.73) (end 130.81 125.73) (width 0.4) (layer F.Cu) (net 16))
 (segment (start 121.92 151.13) (end 116.84 146.05) (width 0.4) (layer F.Cu) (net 16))
 (segment (start 144.78 151.13) (end 121.92 151.13) (width 0.4) (layer F.Cu) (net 16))
 (segment (start 163.83 144.78) (end 163.83 137.16) (width 0.4) (layer F.Cu) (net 16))
 (segment (start 162.56 146.05) (end 163.83 144.78) (width 0.4) (layer F.Cu) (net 16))
 (segment (start 162.56 151.13) (end 162.56 146.05) (width 0.4) (layer F.Cu) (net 16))
 (segment (start 158.75 160.02) (end 171.45 160.02) (width 0.4) (layer F.Cu) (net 16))
 (segment (start 175.26 153.63) (end 175.26 156.21) (width 0.4) (layer F.Cu) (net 16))
 (segment (start 171.45 160.02) (end 184.15 160.02) (width 0.4) (layer F.Cu) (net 16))
 (segment (start 175.26 156.21) (end 171.45 160.02) (width 0.4) (layer F.Cu) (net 16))
 (segment (start 150.275888 160.02) (end 158.75 160.02) (width 0.4) (layer F.Cu) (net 16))
 (segment (start 162.56 151.13) (end 162.56 156.21) (width 0.4) (layer F.Cu) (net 16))
 (segment (start 162.56 156.21) (end 158.75 160.02) (width 0.4) (layer F.Cu) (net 16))
 (segment (start 144.78 58.42) (end 144.78 53.34) (width 0.4) (layer F.Cu) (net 16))
 (segment (start 144.78 53.34) (end 140.97 49.53) (width 0.4) (layer F.Cu) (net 16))
 (segment (start 140.97 49.53) (end 140.97 35.56) (width 0.4) (layer F.Cu) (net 16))
 (segment (start 140.97 35.56) (end 142.24 34.29) (width 0.4) (layer F.Cu) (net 16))
 (segment (start 142.24 34.29) (end 175.26 34.29) (width 0.4) (layer F.Cu) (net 16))
 (segment (start 175.26 34.29) (end 182.88 41.91) (width 0.4) (layer F.Cu) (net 16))
 (segment (start 182.88 41.91) (end 182.88 50.8) (width 0.4) (layer F.Cu) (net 16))
 (segment (start 163.83 67.31) (end 163.83 62.23) (width 0.4) (layer F.Cu) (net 16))
 (segment (start 163.83 62.23) (end 163.83 58.94) (width 0.4) (layer F.Cu) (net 16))
 (segment (start 158.75 55.88) (end 158.75 57.15) (width 0.4) (layer F.Cu) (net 16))
 (segment (start 158.75 57.15) (end 163.83 62.23) (width 0.4) (layer F.Cu) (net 16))
 (segment (start 163.83 58.94) (end 171.97 50.8) (width 0.4) (layer F.Cu) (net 16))
 (segment (start 171.97 50.8) (end 172.72 50.8) (width 0.4) (layer F.Cu) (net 16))
 (segment (start 144.78 151.13) (end 144.78 154.524112) (width 0.4) (layer F.Cu) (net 16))
 (segment (start 144.78 154.524112) (end 150.275888 160.02) (width 0.4) (layer F.Cu) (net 16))
 (segment (start 184.15 160.02) (end 190.5 153.67) (width 0.4) (layer F.Cu) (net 16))
 (segment (start 190.5 58.42) (end 182.88 50.8) (width 0.4) (layer F.Cu) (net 16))
 (segment (start 182.88 50.8) (end 172.72 50.8) (width 0.4) (layer F.Cu) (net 16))
 (segment (start 177.8 76.2) (end 173.99 72.39) (width 0.4) (layer F.Cu) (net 25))
 (segment (start 173.99 72.39) (end 173.99 67.31) (width 0.4) (layer F.Cu) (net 25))
 (segment (start 177.8 90.17) (end 177.8 76.2) (width 0.4) (layer F.Cu) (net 25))
 (segment (start 173.99 93.98) (end 155.98 93.98) (width 0.4) (layer F.Cu) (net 25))
 (segment (start 155.98 93.98) (end 152.32 97.64) (width 0.4) (layer F.Cu) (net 25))
 (segment (start 177.8 95.25) (end 177.8 90.17) (width 0.4) (layer F.Cu) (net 25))
 (segment (start 177.8 90.17) (end 173.99 93.98) (width 0.4) (layer F.Cu) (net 25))
 (segment (start 177.8 99.06) (end 177.8 95.25) (width 0.4) (layer F.Cu) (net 25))
 (segment (start 165.1 151.13) (end 165.1 146.05) (width 0.4) (layer F.Cu) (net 25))
 (segment (start 165.1 146.05) (end 173.99 137.16) (width 0.4) (layer F.Cu) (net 25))
 (segment (start 173.99 137.16) (end 173.99 118.11) (width 0.4) (layer F.Cu) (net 25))
 (segment (start 173.99 118.11) (end 177.8 114.3) (width 0.4) (layer F.Cu) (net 25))
 (segment (start 177.8 114.3) (end 177.8 99.06) (width 0.4) (layer F.Cu) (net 25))
 (segment (start 165.1 151.13) (end 175.26 151.13) (width 0.4) (layer F.Cu) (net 25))
 (segment (start 163.83 44.45) (end 167.64 48.26) (width 0.4) (layer F.Cu) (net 25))
 (segment (start 167.64 48.26) (end 172.72 48.26) (width 0.4) (layer F.Cu) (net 25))
 (segment (start 161.29 44.45) (end 163.83 44.45) (width 0.4) (layer F.Cu) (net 25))
 (segment (start 160.02 45.72) (end 161.29 44.45) (width 0.4) (layer F.Cu) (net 25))
 (segment (start 158.75 49.53) (end 160.02 48.26) (width 0.4) (layer F.Cu) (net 25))
 (segment (start 160.02 48.26) (end 160.02 45.72) (width 0.4) (layer F.Cu) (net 25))
 (segment (start 154.94 39.37) (end 154.94 45.72) (width 0.4) (layer F.Cu) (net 25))
 (segment (start 154.94 45.72) (end 158.75 49.53) (width 0.4) (layer F.Cu) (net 25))
 (segment (start 147.32 97.64) (end 147.32 109.22) (width 0.4) (layer F.Cu) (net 31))
 (segment (start 147.32 109.22) (end 135.89 120.65) (width 0.4) (layer F.Cu) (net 31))
 (segment (start 135.89 120.65) (end 130.81 120.65) (width 0.4) (layer F.Cu) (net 31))
 (segment (start 157.48 116.84) (end 143.51 130.81) (width 0.4) (layer F.Cu) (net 6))
 (segment (start 143.51 130.81) (end 130.81 130.81) (width 0.4) (layer F.Cu) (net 6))
 (segment (start 168.91 116.84) (end 157.48 116.84) (width 0.4) (layer F.Cu) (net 6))
 (segment (start 156.21 119.38) (end 142.24 133.35) (width 0.4) (layer F.Cu) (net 7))
 (segment (start 142.24 133.35) (end 130.81 133.35) (width 0.4) (layer F.Cu) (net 7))
 (segment (start 168.91 119.38) (end 156.21 119.38) (width 0.4) (layer F.Cu) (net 7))
 (segment (start 168.91 121.92) (end 154.94 121.92) (width 0.4) (layer F.Cu) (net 8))
 (segment (start 154.94 121.92) (end 140.97 135.89) (width 0.4) (layer F.Cu) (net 8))
 (segment (start 140.97 135.89) (end 130.81 135.89) (width 0.4) (layer F.Cu) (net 8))
 (segment (start 139.7 138.43) (end 130.81 138.43) (width 0.4) (layer F.Cu) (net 9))
 (segment (start 153.67 124.46) (end 139.7 138.43) (width 0.4) (layer F.Cu) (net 9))
 (segment (start 168.91 124.46) (end 153.67 124.46) (width 0.4) (layer F.Cu) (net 9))
 (segment (start 171.45 67.31) (end 171.45 75.833602) (width 0.4) (layer F.Cu) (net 5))
 (segment (start 171.45 75.833602) (end 149.86 97.423602) (width 0.4) (layer F.Cu) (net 5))
 (segment (start 149.86 97.423602) (end 149.86 106.68) (width 0.4) (layer F.Cu) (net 5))
 (segment (start 149.86 106.68) (end 154.94 111.76) (width 0.4) (layer F.Cu) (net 5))
 (segment (start 154.94 111.76) (end 168.91 111.76) (width 0.4) (layer F.Cu) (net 5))
 (segment (start 161.29 67.31) (end 161.29 68.06) (width 0.4) (layer F.Cu) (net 37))
 (segment (start 161.29 49.53) (end 157.48 53.34) (width 0.4) (layer F.Cu) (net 37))
 (segment (start 157.48 53.34) (end 156.21 54.61) (width 0.4) (layer F.Cu) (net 37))
 (segment (start 161.29 55.88) (end 158.75 53.34) (width 0.4) (layer F.Cu) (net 37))
 (segment (start 158.75 53.34) (end 157.48 53.34) (width 0.4) (layer F.Cu) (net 37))
 (segment (start 156.21 54.61) (end 156.21 61.48) (width 0.4) (layer F.Cu) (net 37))
 (segment (start 156.21 61.48) (end 161.29 66.56) (width 0.4) (layer F.Cu) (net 37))
 (segment (start 161.29 66.56) (end 161.29 67.31) (width 0.4) (layer F.Cu) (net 37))
 (segment (start 147.32 39.37) (end 147.32 58.42) (width 0.4) (layer F.Cu) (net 38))
 (segment (start 176.53 129.54) (end 176.53 129.19075) (width 0.4) (layer F.Cu) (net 22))
 (segment (start 182.88 99.40925) (end 182.88 99.06) (width 0.4) (layer F.Cu) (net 23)))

